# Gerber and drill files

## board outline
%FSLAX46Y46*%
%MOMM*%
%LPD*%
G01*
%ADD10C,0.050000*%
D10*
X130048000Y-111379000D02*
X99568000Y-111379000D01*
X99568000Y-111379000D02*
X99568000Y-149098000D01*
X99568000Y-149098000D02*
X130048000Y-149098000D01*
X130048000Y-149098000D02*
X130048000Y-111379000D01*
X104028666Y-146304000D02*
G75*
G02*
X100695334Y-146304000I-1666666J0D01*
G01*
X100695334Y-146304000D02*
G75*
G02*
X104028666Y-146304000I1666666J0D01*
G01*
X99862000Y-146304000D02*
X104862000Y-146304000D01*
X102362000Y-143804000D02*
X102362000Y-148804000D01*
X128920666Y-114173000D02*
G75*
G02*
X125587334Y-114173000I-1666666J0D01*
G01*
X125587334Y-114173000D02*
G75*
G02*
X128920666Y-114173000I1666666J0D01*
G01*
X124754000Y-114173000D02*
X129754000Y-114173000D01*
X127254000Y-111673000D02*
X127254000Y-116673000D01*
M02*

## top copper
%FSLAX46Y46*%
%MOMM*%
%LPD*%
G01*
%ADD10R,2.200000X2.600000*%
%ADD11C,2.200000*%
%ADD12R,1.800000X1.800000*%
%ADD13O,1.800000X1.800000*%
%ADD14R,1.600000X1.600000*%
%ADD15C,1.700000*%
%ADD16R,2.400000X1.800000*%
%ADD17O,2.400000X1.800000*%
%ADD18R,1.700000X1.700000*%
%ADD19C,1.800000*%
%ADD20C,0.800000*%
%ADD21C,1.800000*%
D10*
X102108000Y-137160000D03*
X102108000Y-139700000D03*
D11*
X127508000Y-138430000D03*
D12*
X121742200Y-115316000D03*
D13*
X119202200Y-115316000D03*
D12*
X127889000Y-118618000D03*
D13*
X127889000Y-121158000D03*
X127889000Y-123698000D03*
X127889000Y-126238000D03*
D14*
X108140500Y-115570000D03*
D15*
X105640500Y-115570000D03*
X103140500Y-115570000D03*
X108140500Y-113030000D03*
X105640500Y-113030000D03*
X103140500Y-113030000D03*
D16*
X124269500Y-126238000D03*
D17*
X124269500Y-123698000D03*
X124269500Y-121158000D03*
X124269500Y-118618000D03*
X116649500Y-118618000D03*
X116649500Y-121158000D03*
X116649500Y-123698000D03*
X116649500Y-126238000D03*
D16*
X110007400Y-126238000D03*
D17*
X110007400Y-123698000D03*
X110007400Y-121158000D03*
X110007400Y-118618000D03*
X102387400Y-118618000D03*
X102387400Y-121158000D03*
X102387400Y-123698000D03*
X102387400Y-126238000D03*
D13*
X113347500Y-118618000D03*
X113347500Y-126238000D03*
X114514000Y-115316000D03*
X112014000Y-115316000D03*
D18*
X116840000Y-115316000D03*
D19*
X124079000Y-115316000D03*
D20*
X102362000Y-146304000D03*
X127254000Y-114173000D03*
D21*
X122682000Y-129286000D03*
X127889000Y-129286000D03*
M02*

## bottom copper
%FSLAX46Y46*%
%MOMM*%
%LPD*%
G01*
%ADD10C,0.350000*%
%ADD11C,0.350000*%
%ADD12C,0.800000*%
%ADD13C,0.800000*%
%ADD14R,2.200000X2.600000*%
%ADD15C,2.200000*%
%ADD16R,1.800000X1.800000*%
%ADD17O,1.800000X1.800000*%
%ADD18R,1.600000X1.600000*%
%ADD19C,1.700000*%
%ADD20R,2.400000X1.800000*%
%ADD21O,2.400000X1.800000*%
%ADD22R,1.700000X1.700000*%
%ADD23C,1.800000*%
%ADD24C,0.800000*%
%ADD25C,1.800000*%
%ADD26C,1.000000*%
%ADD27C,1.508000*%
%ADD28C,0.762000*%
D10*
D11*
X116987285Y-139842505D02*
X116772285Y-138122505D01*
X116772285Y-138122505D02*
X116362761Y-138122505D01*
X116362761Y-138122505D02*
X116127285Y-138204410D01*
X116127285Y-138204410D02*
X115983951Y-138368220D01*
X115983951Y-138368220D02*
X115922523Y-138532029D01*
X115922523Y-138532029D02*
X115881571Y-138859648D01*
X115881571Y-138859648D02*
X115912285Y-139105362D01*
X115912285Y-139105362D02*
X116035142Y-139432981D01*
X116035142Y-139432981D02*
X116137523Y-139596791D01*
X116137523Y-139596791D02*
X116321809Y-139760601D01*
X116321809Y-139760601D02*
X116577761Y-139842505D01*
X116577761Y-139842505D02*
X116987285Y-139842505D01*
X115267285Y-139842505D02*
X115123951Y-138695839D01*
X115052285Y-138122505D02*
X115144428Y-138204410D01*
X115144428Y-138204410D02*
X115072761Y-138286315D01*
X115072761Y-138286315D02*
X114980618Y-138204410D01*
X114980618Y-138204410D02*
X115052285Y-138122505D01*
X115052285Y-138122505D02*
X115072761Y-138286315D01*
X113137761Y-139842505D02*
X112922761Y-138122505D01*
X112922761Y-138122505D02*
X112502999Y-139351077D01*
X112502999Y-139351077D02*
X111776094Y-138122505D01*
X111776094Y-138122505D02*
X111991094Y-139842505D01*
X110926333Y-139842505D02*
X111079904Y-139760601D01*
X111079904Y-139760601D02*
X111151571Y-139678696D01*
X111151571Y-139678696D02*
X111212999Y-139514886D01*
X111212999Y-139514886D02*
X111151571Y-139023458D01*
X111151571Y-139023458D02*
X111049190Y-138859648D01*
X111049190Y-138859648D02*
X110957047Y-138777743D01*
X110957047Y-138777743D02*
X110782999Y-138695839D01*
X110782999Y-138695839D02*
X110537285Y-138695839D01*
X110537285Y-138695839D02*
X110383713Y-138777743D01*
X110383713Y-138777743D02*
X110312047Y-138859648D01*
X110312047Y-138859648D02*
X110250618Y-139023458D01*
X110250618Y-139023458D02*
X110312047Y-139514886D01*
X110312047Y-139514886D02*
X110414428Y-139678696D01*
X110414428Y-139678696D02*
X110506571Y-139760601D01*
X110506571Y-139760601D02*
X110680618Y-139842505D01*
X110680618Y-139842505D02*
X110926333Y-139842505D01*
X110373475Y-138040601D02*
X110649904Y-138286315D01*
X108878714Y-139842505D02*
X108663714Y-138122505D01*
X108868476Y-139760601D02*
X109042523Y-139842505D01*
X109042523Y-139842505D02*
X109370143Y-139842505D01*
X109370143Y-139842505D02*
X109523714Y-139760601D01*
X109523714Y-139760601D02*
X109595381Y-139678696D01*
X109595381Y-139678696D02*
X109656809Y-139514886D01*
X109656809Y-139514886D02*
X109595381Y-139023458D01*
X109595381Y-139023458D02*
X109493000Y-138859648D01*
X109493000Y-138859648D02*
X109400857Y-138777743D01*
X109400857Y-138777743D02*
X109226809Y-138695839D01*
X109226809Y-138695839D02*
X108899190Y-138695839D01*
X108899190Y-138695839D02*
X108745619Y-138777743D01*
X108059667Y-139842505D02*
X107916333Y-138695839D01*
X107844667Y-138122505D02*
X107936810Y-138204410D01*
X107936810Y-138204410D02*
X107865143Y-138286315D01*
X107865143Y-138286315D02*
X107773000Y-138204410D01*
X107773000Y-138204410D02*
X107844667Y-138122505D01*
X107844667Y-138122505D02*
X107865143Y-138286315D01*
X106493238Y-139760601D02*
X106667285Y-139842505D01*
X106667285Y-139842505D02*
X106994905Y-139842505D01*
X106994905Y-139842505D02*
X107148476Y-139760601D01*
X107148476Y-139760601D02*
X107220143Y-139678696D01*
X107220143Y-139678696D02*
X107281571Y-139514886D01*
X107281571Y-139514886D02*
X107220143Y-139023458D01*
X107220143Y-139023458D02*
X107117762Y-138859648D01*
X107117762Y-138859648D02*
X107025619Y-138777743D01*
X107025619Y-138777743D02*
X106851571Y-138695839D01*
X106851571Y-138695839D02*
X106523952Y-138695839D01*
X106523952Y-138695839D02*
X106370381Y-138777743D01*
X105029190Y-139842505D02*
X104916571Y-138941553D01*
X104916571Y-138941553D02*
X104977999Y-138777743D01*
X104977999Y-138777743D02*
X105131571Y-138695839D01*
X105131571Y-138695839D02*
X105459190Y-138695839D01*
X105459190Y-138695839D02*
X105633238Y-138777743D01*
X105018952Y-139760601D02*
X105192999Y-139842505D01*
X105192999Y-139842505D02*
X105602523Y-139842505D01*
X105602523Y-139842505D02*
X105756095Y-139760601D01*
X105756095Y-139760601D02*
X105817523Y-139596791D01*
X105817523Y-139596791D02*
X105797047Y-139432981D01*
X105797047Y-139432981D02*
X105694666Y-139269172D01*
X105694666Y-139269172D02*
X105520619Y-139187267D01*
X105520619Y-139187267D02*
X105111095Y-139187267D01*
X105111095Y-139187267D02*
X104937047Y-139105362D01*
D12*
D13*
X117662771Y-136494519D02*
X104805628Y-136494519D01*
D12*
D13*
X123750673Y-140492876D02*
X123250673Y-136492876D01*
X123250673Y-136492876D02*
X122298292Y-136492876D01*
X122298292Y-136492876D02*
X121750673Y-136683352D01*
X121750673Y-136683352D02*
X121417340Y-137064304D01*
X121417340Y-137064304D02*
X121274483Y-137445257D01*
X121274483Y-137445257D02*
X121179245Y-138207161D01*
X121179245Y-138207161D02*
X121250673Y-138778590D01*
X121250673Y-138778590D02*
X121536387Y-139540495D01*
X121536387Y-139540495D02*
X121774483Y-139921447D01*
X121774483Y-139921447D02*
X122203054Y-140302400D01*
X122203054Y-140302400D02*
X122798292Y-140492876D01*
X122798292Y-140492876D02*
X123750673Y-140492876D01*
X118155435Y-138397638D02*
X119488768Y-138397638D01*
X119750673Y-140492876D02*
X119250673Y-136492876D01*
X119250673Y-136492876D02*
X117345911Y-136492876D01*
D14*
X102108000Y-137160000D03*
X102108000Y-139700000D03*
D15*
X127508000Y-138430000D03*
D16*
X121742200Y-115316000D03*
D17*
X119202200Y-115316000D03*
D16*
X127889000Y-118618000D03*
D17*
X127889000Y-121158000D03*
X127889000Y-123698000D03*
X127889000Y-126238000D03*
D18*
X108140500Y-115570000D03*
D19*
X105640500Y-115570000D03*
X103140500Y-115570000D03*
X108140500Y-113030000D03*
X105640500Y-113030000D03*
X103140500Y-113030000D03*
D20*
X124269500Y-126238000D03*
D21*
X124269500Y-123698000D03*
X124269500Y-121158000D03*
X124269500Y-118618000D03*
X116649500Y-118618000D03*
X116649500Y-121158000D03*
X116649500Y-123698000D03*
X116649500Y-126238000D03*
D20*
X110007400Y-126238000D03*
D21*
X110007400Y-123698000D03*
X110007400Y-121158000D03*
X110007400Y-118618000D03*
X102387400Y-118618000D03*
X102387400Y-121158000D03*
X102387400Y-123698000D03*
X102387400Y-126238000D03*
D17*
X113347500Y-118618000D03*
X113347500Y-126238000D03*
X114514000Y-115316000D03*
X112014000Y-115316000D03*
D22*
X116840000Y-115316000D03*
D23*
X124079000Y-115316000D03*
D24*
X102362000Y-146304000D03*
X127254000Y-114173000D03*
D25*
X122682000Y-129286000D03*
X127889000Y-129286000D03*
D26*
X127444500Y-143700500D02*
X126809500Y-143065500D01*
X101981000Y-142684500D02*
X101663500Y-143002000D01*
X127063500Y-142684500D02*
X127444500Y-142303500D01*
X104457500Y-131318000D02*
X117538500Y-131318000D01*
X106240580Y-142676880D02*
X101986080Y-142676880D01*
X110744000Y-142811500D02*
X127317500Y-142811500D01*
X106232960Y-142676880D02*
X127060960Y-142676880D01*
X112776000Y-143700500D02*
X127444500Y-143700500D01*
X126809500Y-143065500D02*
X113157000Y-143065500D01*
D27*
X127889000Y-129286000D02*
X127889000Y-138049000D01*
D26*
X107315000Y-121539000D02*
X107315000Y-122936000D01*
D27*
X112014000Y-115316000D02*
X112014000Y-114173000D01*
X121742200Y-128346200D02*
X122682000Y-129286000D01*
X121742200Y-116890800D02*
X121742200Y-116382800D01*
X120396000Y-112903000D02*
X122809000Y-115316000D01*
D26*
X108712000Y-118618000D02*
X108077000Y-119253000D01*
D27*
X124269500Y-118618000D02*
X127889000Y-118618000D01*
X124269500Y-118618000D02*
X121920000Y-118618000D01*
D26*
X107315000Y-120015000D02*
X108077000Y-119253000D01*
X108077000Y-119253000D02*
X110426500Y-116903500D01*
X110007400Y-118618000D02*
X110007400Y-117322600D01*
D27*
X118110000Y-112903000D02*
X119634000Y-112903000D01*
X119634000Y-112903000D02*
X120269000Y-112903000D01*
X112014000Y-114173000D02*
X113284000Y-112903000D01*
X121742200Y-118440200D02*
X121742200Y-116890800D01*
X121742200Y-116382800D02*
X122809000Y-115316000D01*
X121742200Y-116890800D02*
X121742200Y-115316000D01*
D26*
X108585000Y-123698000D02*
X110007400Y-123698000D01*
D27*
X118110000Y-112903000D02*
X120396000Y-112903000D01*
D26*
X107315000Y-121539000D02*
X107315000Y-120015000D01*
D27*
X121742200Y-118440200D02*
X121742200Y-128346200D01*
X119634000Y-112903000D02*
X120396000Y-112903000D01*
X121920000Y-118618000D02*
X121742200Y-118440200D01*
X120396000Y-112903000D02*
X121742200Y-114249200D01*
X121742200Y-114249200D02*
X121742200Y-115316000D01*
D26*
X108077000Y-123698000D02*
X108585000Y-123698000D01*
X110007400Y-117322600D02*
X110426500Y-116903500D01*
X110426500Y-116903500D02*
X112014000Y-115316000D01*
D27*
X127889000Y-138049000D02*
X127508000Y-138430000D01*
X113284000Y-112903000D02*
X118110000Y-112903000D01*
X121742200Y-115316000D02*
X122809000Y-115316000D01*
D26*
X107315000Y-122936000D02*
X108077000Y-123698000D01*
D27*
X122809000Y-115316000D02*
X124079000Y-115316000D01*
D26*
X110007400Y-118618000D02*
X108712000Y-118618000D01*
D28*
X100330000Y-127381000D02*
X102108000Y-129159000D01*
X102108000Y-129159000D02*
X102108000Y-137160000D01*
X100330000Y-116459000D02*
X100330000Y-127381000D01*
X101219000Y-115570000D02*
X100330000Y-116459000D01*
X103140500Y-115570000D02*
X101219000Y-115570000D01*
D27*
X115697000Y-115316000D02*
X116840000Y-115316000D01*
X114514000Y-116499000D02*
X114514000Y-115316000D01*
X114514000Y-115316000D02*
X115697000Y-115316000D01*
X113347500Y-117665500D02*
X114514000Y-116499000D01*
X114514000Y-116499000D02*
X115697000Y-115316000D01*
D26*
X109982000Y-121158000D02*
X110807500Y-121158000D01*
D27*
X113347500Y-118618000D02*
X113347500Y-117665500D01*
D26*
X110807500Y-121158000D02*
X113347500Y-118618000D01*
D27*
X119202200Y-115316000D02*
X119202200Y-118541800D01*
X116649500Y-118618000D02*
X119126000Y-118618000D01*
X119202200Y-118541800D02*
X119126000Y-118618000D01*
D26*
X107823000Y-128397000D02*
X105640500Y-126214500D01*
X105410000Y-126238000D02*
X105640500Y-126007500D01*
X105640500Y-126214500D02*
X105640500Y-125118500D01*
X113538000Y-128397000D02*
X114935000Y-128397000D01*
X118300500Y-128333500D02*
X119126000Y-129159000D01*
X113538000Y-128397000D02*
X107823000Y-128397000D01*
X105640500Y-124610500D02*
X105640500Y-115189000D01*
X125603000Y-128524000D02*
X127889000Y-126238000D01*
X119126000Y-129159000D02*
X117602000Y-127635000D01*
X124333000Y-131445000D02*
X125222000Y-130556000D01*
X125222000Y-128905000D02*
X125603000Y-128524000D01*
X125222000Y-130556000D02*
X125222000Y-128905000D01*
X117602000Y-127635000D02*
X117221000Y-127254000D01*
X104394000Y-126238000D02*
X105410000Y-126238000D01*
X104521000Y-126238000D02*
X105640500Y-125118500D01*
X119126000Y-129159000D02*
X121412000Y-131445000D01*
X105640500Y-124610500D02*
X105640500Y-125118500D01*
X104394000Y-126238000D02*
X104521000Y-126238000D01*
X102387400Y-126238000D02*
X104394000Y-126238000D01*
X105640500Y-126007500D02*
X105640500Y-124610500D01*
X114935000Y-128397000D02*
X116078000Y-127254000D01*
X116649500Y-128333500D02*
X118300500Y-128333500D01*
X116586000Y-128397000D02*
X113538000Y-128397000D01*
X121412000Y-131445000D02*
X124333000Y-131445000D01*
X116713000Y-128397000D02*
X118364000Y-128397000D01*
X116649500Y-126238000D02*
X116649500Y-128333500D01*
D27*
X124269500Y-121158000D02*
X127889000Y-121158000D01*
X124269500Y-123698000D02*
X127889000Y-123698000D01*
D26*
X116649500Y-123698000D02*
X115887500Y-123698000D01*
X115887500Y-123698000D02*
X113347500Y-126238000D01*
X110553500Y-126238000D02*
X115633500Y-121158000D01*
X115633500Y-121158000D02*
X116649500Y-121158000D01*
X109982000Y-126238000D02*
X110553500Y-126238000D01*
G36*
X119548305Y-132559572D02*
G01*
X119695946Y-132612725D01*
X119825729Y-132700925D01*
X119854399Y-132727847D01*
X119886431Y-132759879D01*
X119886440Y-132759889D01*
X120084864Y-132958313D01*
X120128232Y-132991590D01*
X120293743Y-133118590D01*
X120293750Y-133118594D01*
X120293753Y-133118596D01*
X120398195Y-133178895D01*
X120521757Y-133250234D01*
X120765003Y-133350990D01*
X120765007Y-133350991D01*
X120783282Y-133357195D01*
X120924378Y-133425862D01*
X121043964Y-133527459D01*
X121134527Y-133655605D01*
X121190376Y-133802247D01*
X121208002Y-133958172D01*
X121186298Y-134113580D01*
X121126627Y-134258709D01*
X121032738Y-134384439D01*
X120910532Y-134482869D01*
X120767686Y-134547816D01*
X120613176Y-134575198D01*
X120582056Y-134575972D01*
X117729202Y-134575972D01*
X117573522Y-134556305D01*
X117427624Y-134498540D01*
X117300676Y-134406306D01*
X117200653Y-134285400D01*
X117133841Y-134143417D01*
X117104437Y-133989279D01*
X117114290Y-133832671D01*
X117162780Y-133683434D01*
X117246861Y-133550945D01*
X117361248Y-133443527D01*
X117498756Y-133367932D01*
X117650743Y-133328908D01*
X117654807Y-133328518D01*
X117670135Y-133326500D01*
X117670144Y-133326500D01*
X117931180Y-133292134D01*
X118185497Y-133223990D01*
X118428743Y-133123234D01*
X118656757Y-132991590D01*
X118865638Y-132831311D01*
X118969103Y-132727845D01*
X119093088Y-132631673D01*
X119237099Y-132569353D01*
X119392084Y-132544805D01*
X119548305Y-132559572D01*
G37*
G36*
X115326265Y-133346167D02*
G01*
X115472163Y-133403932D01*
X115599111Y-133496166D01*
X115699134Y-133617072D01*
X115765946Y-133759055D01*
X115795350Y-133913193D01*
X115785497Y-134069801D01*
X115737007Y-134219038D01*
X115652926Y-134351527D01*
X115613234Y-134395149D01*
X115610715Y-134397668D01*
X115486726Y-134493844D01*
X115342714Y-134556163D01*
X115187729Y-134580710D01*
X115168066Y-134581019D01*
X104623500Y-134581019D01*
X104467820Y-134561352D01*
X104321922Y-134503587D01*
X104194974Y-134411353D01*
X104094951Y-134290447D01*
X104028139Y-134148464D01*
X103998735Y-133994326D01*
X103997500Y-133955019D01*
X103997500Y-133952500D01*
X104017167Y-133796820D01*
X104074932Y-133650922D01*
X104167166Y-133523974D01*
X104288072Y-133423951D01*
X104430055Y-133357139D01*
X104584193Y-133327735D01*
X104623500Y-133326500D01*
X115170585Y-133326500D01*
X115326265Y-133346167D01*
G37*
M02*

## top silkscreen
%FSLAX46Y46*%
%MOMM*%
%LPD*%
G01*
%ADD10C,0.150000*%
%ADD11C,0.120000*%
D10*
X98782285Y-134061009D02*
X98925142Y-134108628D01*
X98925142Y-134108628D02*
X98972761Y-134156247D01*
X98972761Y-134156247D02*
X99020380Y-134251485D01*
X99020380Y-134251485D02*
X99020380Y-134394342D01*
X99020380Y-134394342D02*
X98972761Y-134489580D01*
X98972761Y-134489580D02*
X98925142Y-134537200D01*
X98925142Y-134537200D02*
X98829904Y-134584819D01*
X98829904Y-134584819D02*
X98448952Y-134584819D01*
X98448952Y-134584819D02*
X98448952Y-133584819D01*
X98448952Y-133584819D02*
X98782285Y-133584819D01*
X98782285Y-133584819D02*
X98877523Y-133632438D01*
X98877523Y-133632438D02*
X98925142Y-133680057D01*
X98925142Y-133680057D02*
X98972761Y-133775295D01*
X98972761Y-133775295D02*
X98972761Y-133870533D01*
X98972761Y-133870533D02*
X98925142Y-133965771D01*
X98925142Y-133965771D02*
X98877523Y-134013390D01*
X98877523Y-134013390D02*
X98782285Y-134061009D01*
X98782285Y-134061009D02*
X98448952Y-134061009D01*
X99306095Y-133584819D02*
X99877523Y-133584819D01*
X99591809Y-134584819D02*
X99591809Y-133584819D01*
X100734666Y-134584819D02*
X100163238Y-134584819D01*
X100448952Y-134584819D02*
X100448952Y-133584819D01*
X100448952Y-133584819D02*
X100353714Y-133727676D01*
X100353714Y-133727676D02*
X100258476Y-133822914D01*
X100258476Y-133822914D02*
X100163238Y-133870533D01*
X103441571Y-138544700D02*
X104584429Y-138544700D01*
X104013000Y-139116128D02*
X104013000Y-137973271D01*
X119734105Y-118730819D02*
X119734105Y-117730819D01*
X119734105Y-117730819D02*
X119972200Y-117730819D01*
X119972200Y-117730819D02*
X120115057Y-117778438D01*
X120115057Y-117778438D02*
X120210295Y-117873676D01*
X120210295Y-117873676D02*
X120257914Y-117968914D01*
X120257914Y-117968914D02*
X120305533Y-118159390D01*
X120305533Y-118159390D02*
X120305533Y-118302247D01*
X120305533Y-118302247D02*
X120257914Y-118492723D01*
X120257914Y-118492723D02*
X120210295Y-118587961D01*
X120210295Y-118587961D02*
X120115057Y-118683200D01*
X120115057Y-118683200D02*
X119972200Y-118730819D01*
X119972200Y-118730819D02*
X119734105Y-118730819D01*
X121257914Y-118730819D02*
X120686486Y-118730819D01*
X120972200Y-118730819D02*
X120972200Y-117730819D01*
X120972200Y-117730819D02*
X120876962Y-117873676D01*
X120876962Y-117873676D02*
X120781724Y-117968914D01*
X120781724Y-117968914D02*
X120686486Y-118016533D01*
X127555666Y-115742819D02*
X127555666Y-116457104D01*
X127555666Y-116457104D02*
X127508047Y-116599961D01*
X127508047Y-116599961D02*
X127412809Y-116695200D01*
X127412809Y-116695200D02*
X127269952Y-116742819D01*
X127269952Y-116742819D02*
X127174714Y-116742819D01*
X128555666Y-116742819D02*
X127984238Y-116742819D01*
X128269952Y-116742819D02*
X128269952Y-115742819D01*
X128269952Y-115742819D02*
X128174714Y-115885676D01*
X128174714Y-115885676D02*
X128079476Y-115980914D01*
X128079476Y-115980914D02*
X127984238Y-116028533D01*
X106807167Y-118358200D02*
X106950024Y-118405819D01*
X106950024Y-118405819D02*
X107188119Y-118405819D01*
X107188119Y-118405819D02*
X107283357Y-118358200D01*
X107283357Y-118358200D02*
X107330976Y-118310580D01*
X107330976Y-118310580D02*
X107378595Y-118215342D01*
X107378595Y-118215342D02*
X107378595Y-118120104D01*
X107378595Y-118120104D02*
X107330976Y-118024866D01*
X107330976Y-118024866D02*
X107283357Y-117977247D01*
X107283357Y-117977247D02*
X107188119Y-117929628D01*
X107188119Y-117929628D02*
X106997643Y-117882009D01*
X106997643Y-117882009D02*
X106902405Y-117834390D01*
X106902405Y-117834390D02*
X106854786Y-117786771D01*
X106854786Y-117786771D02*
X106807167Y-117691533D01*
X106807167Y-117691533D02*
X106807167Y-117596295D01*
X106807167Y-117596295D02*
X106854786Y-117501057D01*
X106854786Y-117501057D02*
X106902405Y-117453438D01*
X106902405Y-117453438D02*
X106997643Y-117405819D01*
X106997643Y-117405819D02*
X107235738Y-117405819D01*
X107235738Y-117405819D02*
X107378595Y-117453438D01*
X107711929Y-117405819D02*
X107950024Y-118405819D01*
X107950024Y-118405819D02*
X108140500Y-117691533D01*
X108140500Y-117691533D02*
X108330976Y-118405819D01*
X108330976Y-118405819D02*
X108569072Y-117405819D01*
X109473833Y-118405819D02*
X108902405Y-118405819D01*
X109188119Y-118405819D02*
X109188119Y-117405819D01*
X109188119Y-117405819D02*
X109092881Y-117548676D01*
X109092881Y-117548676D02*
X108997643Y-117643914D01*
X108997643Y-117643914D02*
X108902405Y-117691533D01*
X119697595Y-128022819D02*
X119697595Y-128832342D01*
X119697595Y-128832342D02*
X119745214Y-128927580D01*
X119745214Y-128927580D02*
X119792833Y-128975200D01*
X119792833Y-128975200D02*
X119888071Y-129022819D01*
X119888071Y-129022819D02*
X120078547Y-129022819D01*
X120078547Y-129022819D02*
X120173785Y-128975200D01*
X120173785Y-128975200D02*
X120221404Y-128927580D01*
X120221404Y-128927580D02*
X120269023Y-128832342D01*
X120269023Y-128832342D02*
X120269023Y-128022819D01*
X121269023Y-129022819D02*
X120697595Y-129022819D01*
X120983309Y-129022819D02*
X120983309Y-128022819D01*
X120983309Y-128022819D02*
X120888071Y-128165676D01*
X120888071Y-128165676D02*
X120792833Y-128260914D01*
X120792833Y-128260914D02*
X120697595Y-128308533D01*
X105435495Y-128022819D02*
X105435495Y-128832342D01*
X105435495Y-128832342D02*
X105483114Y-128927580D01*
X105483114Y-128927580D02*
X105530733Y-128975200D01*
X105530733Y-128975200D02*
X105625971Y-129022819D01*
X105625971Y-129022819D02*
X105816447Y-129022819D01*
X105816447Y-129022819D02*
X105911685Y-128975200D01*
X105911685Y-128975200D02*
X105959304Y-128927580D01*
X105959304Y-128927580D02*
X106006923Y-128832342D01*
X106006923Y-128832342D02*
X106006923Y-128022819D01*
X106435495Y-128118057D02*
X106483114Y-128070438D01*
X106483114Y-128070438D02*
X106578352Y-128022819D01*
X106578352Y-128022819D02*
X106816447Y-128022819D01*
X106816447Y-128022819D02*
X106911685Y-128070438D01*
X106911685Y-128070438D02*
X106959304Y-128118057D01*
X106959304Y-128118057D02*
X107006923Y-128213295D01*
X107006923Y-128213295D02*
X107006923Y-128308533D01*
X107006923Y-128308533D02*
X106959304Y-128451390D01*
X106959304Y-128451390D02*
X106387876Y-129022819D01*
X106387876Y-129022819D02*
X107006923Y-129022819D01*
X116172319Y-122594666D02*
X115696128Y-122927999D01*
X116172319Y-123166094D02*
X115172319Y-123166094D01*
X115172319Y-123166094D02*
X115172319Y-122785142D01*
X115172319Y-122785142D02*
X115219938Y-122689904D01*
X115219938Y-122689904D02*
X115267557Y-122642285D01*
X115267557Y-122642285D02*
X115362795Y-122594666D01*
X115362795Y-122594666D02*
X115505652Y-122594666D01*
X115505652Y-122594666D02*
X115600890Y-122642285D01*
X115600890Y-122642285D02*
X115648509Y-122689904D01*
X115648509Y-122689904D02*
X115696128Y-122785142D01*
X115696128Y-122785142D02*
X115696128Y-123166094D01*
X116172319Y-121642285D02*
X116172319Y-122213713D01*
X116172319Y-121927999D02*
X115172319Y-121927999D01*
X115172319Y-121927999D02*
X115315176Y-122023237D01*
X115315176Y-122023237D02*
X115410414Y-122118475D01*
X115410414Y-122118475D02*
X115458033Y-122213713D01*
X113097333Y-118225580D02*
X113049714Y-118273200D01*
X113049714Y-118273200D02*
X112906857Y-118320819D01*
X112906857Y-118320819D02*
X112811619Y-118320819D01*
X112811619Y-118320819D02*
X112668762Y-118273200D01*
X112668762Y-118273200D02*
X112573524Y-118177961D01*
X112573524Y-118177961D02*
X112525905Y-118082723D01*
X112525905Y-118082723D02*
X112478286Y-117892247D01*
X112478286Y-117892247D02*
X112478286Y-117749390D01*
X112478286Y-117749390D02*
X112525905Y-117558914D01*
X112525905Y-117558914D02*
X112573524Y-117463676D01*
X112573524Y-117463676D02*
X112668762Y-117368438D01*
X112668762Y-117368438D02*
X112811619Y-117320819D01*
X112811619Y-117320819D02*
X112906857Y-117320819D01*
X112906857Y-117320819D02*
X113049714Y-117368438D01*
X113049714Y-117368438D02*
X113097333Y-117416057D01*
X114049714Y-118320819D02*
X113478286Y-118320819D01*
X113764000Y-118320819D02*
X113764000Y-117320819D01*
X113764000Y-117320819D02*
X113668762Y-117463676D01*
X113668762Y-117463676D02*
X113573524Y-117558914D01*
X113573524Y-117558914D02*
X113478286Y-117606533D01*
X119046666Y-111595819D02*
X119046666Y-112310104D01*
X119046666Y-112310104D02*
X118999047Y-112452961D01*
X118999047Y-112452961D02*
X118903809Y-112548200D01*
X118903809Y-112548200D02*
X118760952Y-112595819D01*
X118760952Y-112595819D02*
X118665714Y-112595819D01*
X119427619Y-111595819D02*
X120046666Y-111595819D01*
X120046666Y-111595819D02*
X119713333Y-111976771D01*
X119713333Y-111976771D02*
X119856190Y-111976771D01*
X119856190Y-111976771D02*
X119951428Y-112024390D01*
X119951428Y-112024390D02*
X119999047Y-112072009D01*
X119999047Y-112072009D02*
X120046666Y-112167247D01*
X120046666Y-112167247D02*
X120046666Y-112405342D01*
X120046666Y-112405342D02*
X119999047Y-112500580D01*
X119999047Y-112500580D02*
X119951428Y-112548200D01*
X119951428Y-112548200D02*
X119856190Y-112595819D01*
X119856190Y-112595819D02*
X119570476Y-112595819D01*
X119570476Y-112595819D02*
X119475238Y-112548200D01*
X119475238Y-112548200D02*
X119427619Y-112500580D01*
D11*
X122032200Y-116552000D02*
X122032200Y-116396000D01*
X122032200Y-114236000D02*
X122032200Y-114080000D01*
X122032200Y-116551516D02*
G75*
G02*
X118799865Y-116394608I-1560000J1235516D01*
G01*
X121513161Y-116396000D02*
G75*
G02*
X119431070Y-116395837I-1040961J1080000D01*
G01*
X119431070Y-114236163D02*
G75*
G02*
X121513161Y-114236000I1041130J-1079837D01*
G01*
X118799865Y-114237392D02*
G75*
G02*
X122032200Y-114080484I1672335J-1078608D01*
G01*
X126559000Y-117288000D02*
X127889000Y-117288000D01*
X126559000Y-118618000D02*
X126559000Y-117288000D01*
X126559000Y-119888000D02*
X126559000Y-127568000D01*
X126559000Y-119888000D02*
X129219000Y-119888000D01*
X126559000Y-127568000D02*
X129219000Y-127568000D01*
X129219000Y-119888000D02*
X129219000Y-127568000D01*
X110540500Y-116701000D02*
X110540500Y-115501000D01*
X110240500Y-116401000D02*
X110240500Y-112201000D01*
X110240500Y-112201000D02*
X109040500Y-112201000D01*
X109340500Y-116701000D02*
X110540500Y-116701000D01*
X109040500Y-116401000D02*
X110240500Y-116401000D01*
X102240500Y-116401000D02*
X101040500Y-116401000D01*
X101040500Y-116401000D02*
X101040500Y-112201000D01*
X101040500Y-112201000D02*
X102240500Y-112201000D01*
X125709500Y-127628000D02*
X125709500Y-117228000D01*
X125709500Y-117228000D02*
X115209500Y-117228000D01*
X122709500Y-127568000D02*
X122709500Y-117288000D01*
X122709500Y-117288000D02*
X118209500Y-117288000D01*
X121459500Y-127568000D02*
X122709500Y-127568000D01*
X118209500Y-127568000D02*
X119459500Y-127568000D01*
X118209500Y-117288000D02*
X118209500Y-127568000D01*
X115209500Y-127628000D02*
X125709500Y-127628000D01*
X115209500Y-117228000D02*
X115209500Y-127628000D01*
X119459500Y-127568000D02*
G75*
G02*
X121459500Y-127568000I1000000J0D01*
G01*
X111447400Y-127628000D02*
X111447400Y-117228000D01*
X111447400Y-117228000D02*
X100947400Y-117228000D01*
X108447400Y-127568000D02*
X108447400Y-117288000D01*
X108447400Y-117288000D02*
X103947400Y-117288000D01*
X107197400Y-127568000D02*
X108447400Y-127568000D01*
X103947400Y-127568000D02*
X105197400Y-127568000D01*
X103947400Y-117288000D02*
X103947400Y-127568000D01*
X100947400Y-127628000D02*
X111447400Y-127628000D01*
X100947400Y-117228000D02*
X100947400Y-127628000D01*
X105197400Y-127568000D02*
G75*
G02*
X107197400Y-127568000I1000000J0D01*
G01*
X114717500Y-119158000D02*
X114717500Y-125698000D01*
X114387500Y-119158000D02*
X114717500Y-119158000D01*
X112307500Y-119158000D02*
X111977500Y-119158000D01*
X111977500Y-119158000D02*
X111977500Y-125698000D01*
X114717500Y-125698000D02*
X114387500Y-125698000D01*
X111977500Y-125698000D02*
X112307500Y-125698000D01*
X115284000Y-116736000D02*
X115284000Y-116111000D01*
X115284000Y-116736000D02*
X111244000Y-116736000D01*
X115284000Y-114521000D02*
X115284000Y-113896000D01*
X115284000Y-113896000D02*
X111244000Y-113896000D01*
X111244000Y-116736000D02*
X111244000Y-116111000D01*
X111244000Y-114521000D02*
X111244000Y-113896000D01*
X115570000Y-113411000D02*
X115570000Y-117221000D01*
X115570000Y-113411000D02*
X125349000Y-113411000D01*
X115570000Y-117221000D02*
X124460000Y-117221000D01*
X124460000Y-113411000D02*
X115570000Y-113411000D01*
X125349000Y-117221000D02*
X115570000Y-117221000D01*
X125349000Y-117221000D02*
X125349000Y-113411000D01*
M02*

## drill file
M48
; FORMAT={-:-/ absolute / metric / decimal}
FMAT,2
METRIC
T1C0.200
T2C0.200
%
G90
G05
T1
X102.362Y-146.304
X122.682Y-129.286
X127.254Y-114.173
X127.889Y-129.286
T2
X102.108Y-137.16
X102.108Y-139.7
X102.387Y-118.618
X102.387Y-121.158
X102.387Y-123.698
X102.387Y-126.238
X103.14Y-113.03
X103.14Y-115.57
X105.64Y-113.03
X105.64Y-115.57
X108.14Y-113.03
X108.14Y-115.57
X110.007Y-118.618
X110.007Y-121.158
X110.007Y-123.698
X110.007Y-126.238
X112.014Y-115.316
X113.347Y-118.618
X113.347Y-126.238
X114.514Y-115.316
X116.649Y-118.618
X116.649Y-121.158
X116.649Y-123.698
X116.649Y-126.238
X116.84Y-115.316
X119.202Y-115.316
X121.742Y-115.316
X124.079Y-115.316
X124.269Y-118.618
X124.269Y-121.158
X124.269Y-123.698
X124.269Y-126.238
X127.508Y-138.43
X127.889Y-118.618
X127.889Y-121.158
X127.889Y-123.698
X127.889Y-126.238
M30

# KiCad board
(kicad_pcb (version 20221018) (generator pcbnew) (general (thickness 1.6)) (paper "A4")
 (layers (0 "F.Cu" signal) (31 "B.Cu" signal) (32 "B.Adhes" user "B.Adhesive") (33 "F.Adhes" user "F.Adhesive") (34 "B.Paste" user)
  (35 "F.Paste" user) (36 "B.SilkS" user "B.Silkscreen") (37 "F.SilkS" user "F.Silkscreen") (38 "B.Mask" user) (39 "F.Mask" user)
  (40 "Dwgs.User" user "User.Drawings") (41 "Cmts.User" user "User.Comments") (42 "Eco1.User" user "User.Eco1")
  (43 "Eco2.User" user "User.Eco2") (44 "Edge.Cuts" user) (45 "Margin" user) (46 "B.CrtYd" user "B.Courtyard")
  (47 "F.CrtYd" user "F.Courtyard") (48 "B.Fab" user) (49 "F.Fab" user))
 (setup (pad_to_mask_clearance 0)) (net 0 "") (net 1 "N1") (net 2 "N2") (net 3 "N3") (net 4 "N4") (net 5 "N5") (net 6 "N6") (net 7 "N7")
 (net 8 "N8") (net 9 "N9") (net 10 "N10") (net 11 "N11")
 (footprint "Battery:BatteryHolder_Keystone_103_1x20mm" (layer "F.Cu") (at 99.568 138.43)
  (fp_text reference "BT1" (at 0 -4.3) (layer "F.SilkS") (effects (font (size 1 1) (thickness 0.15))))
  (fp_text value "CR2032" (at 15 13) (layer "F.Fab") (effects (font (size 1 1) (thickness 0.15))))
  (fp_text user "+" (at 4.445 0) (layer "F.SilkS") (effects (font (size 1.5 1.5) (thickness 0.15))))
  (pad "1" thru_hole rect (at 2.54 -1.27) (size 2.2 2.6) (drill 0.2) (layers "*.Cu" "*.Mask") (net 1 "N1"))
  (pad "1" thru_hole rect (at 2.54 1.27) (size 2.2 2.6) (drill 0.2) (layers "*.Cu" "*.Mask") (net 1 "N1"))
  (pad "2" thru_hole circle (at 27.94 0) (size 2.2 2.2) (drill 0.2) (layers "*.Cu" "*.Mask") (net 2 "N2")))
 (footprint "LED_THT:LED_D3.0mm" (layer "F.Cu") (at 121.7422 115.316 180)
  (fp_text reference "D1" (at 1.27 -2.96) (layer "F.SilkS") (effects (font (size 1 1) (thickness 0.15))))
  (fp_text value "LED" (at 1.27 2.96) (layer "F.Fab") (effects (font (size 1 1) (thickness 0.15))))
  (fp_line (start -0.29 -1.236) (end -0.29 -1.08) (stroke (width 0.12) (type solid)) (layer "F.SilkS"))
  (fp_line (start -0.29 1.08) (end -0.29 1.236) (stroke (width 0.12) (type solid)) (layer "F.SilkS"))
  (fp_arc (start -0.29 -1.235516) (mid 1.366487 -1.987659) (end 2.942335 -1.078608) (stroke (width 0.12) (type solid)) (layer "F.SilkS"))
  (fp_arc (start 0.229039 -1.08) (mid 1.270117 -1.5) (end 2.31113 -1.079837) (stroke (width 0.12) (type solid)) (layer "F.SilkS"))
  (fp_arc (start 2.31113 1.079837) (mid 1.270117 1.5) (end 0.229039 1.08) (stroke (width 0.12) (type solid)) (layer "F.SilkS"))
  (fp_arc (start 2.942335 1.078608) (mid 1.366487 1.987659) (end -0.29 1.235516) (stroke (width 0.12) (type solid)) (layer "F.SilkS"))
  (pad "1" thru_hole rect (at 0 0 180) (size 1.8 1.8) (drill 0.2) (layers "*.Cu" "*.Mask") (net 2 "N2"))
  (pad "2" thru_hole oval (at 2.54 0 180) (size 1.8 1.8) (drill 0.2) (layers "*.Cu" "*.Mask") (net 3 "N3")))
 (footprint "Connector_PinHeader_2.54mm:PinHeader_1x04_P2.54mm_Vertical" (layer "F.Cu") (at 127.889 118.618)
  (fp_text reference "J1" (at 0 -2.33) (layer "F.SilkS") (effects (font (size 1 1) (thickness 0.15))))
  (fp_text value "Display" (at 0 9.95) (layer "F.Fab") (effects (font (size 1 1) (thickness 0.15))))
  (fp_line (start -1.33 -1.33) (end 0 -1.33) (stroke (width 0.12) (type solid)) (layer "F.SilkS"))
  (fp_line (start -1.33 0) (end -1.33 -1.33) (stroke (width 0.12) (type solid)) (layer "F.SilkS"))
  (fp_line (start -1.33 1.27) (end -1.33 8.95) (stroke (width 0.12) (type solid)) (layer "F.SilkS"))
  (fp_line (start -1.33 1.27) (end 1.33 1.27) (stroke (width 0.12) (type solid)) (layer "F.SilkS"))
  (fp_line (start -1.33 8.95) (end 1.33 8.95) (stroke (width 0.12) (type solid)) (layer "F.SilkS"))
  (fp_line (start 1.33 1.27) (end 1.33 8.95) (stroke (width 0.12) (type solid)) (layer "F.SilkS"))
  (pad "1" thru_hole rect (at 0 0) (size 1.8 1.8) (drill 0.2) (layers "*.Cu" "*.Mask") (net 2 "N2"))
  (pad "2" thru_hole oval (at 0 2.54) (size 1.8 1.8) (drill 0.2) (layers "*.Cu" "*.Mask") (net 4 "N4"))
  (pad "3" thru_hole oval (at 0 5.08) (size 1.8 1.8) (drill 0.2) (layers "*.Cu" "*.Mask") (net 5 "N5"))
  (pad "4" thru_hole oval (at 0 7.62) (size 1.8 1.8) (drill 0.2) (layers "*.Cu" "*.Mask") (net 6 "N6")))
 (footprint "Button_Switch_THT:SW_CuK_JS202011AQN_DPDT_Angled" (layer "F.Cu") (at 108.1405 115.951 180)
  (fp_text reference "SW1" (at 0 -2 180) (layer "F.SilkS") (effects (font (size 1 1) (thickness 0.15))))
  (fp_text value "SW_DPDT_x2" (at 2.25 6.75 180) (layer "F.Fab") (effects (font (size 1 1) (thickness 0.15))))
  (fp_line (start -2.4 -0.75) (end -2.4 0.45) (stroke (width 0.12) (type solid)) (layer "F.SilkS"))
  (fp_line (start -2.1 -0.45) (end -2.1 3.75) (stroke (width 0.12) (type solid)) (layer "F.SilkS"))
  (fp_line (start -2.1 3.75) (end -0.9 3.75) (stroke (width 0.12) (type solid)) (layer "F.SilkS"))
  (fp_line (start -1.2 -0.75) (end -2.4 -0.75) (stroke (width 0.12) (type solid)) (layer "F.SilkS"))
  (fp_line (start -0.9 -0.45) (end -2.1 -0.45) (stroke (width 0.12) (type solid)) (layer "F.SilkS"))
  (fp_line (start 5.9 -0.45) (end 7.1 -0.45) (stroke (width 0.12) (type solid)) (layer "F.SilkS"))
  (fp_line (start 7.1 -0.45) (end 7.1 3.75) (stroke (width 0.12) (type solid)) (layer "F.SilkS"))
  (fp_line (start 7.1 3.75) (end 5.9 3.75) (stroke (width 0.12) (type solid)) (layer "F.SilkS"))
  (pad "1" thru_hole rect (at 0 0.381 180) (size 1.6 1.6) (drill 0.2) (layers "*.Cu" "*.Mask") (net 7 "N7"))
  (pad "2" thru_hole circle (at 2.5 0.381 180) (size 1.7 1.7) (drill 0.2) (layers "*.Cu" "*.Mask") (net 6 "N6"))
  (pad "3" thru_hole circle (at 5 0.381 180) (size 1.7 1.7) (drill 0.2) (layers "*.Cu" "*.Mask") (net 1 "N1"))
  (pad "4" thru_hole circle (at 0 2.921 180) (size 1.7 1.7) (drill 0.2) (layers "*.Cu" "*.Mask"))
  (pad "5" thru_hole circle (at 2.5 2.921 180) (size 1.7 1.7) (drill 0.2) (layers "*.Cu" "*.Mask"))
  (pad "6" thru_hole circle (at 5 2.921 180) (size 1.7 1.7) (drill 0.2) (layers "*.Cu" "*.Mask")))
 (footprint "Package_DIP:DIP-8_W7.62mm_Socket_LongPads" (layer "F.Cu") (at 124.2695 126.238 180)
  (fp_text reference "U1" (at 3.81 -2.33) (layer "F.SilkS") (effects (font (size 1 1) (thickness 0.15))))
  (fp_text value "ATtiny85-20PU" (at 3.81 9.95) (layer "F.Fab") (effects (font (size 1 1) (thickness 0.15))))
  (fp_line (start -1.44 -1.39) (end -1.44 9.01) (stroke (width 0.12) (type solid)) (layer "F.SilkS"))
  (fp_line (start -1.44 9.01) (end 9.06 9.01) (stroke (width 0.12) (type solid)) (layer "F.SilkS"))
  (fp_line (start 1.56 -1.33) (end 1.56 8.95) (stroke (width 0.12) (type solid)) (layer "F.SilkS"))
  (fp_line (start 1.56 8.95) (end 6.06 8.95) (stroke (width 0.12) (type solid)) (layer "F.SilkS"))
  (fp_line (start 2.81 -1.33) (end 1.56 -1.33) (stroke (width 0.12) (type solid)) (layer "F.SilkS"))
  (fp_line (start 6.06 -1.33) (end 4.81 -1.33) (stroke (width 0.12) (type solid)) (layer "F.SilkS"))
  (fp_line (start 6.06 8.95) (end 6.06 -1.33) (stroke (width 0.12) (type solid)) (layer "F.SilkS"))
  (fp_line (start 9.06 -1.39) (end -1.44 -1.39) (stroke (width 0.12) (type solid)) (layer "F.SilkS"))
  (fp_line (start 9.06 9.01) (end 9.06 -1.39) (stroke (width 0.12) (type solid)) (layer "F.SilkS"))
  (fp_arc (start 4.81 -1.33) (mid 3.81 -0.33) (end 2.81 -1.33) (stroke (width 0.12) (type solid)) (layer "F.SilkS"))
  (pad "1" thru_hole rect (at 0 0 180) (size 2.4 1.8) (drill 0.2) (layers "*.Cu" "*.Mask") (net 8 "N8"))
  (pad "2" thru_hole oval (at 0 2.54 180) (size 2.4 1.8) (drill 0.2) (layers "*.Cu" "*.Mask") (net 5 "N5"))
  (pad "3" thru_hole oval (at 0 5.08 180) (size 2.4 1.8) (drill 0.2) (layers "*.Cu" "*.Mask") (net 4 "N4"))
  (pad "4" thru_hole oval (at 0 7.62 180) (size 2.4 1.8) (drill 0.2) (layers "*.Cu" "*.Mask") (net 2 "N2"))
  (pad "5" thru_hole oval (at 7.62 7.62 180) (size 2.4 1.8) (drill 0.2) (layers "*.Cu" "*.Mask") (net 3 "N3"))
  (pad "6" thru_hole oval (at 7.62 5.08 180) (size 2.4 1.8) (drill 0.2) (layers "*.Cu" "*.Mask") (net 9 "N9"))
  (pad "7" thru_hole oval (at 7.62 2.54 180) (size 2.4 1.8) (drill 0.2) (layers "*.Cu" "*.Mask") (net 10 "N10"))
  (pad "8" thru_hole oval (at 7.62 0 180) (size 2.4 1.8) (drill 0.2) (layers "*.Cu" "*.Mask") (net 6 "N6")))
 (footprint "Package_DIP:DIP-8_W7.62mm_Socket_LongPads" (layer "F.Cu") (at 110.0074 126.238 180)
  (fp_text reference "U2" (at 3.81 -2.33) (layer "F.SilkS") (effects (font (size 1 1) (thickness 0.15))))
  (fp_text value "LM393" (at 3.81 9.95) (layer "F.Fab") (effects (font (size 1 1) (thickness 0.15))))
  (fp_line (start -1.44 -1.39) (end -1.44 9.01) (stroke (width 0.12) (type solid)) (layer "F.SilkS"))
  (fp_line (start -1.44 9.01) (end 9.06 9.01) (stroke (width 0.12) (type solid)) (layer "F.SilkS"))
  (fp_line (start 1.56 -1.33) (end 1.56 8.95) (stroke (width 0.12) (type solid)) (layer "F.SilkS"))
  (fp_line (start 1.56 8.95) (end 6.06 8.95) (stroke (width 0.12) (type solid)) (layer "F.SilkS"))
  (fp_line (start 2.81 -1.33) (end 1.56 -1.33) (stroke (width 0.12) (type solid)) (layer "F.SilkS"))
  (fp_line (start 6.06 -1.33) (end 4.81 -1.33) (stroke (width 0.12) (type solid)) (layer "F.SilkS"))
  (fp_line (start 6.06 8.95) (end 6.06 -1.33) (stroke (width 0.12) (type solid)) (layer "F.SilkS"))
  (fp_line (start 9.06 -1.39) (end -1.44 -1.39) (stroke (width 0.12) (type solid)) (layer "F.SilkS"))
  (fp_line (start 9.06 9.01) (end 9.06 -1.39) (stroke (width 0.12) (type solid)) (layer "F.SilkS"))
  (fp_arc (start 4.81 -1.33) (mid 3.81 -0.33) (end 2.81 -1.33) (stroke (width 0.12) (type solid)) (layer "F.SilkS"))
  (pad "1" thru_hole rect (at 0 0 180) (size 2.4 1.8) (drill 0.2) (layers "*.Cu" "*.Mask") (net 9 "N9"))
  (pad "2" thru_hole oval (at 0 2.54 180) (size 2.4 1.8) (drill 0.2) (layers "*.Cu" "*.Mask") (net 2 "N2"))
  (pad "3" thru_hole oval (at 0 5.08 180) (size 2.4 1.8) (drill 0.2) (layers "*.Cu" "*.Mask") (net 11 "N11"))
  (pad "4" thru_hole oval (at 0 7.62 180) (size 2.4 1.8) (drill 0.2) (layers "*.Cu" "*.Mask") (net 2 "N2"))
  (pad "5" thru_hole oval (at 7.62 7.62 180) (size 2.4 1.8) (drill 0.2) (layers "*.Cu" "*.Mask"))
  (pad "6" thru_hole oval (at 7.62 5.08 180) (size 2.4 1.8) (drill 0.2) (layers "*.Cu" "*.Mask"))
  (pad "7" thru_hole oval (at 7.62 2.54 180) (size 2.4 1.8) (drill 0.2) (layers "*.Cu" "*.Mask"))
  (pad "8" thru_hole oval (at 7.62 0 180) (size 2.4 1.8) (drill 0.2) (layers "*.Cu" "*.Mask") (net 6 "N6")))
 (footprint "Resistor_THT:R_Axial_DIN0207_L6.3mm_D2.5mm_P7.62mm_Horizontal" (layer "F.Cu") (at 113.3475 118.618 -90)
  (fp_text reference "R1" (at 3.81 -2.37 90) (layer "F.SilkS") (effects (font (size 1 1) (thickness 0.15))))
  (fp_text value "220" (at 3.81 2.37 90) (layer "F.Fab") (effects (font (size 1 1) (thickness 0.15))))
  (fp_line (start 0.54 -1.37) (end 7.08 -1.37) (stroke (width 0.12) (type solid)) (layer "F.SilkS"))
  (fp_line (start 0.54 -1.04) (end 0.54 -1.37) (stroke (width 0.12) (type solid)) (layer "F.SilkS"))
  (fp_line (start 0.54 1.04) (end 0.54 1.37) (stroke (width 0.12) (type solid)) (layer "F.SilkS"))
  (fp_line (start 0.54 1.37) (end 7.08 1.37) (stroke (width 0.12) (type solid)) (layer "F.SilkS"))
  (fp_line (start 7.08 -1.37) (end 7.08 -1.04) (stroke (width 0.12) (type solid)) (layer "F.SilkS"))
  (fp_line (start 7.08 1.37) (end 7.08 1.04) (stroke (width 0.12) (type solid)) (layer "F.SilkS"))
  (pad "1" thru_hole oval (at 0 0 270) (size 1.8 1.8) (drill 0.2) (layers "*.Cu" "*.Mask") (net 11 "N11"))
  (pad "2" thru_hole oval (at 7.62 0 270) (size 1.8 1.8) (drill 0.2) (layers "*.Cu" "*.Mask") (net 10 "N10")))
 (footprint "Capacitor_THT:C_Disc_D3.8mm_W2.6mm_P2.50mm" (layer "F.Cu") (at 114.514 115.316 180)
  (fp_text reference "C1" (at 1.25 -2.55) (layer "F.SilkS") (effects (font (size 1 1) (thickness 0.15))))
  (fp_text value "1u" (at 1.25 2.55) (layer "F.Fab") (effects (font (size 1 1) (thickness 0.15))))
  (fp_line (start -0.77 -1.42) (end -0.77 -0.795) (stroke (width 0.12) (type solid)) (layer "F.SilkS"))
  (fp_line (start -0.77 -1.42) (end 3.27 -1.42) (stroke (width 0.12) (type solid)) (layer "F.SilkS"))
  (fp_line (start -0.77 0.795) (end -0.77 1.42) (stroke (width 0.12) (type solid)) (layer "F.SilkS"))
  (fp_line (start -0.77 1.42) (end 3.27 1.42) (stroke (width 0.12) (type solid)) (layer "F.SilkS"))
  (fp_line (start 3.27 -1.42) (end 3.27 -0.795) (stroke (width 0.12) (type solid)) (layer "F.SilkS"))
  (fp_line (start 3.27 0.795) (end 3.27 1.42) (stroke (width 0.12) (type solid)) (layer "F.SilkS"))
  (pad "1" thru_hole oval (at 0 0 180) (size 1.8 1.8) (drill 0.2) (layers "*.Cu" "*.Mask") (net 11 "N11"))
  (pad "2" thru_hole oval (at 2.5 0 180) (size 1.8 1.8) (drill 0.2) (layers "*.Cu" "*.Mask") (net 2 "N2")))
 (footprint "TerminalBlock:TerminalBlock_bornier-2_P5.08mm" (layer "F.Cu") (at 116.84 115.316)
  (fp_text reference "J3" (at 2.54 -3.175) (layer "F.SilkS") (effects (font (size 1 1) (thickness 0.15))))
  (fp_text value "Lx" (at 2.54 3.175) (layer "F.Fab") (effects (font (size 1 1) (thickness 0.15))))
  (fp_line (start -1.27 -1.905) (end -1.27 1.905) (stroke (width 0.12) (type solid)) (layer "F.SilkS"))
  (fp_line (start -1.27 -1.905) (end 8.509 -1.905) (stroke (width 0.12) (type solid)) (layer "F.SilkS"))
  (fp_line (start -1.27 1.905) (end 7.62 1.905) (stroke (width 0.12) (type solid)) (layer "F.SilkS"))
  (fp_line (start 7.62 -1.905) (end -1.27 -1.905) (stroke (width 0.12) (type solid)) (layer "F.SilkS"))
  (fp_line (start 8.509 1.905) (end -1.27 1.905) (stroke (width 0.12) (type solid)) (layer "F.SilkS"))
  (fp_line (start 8.509 1.905) (end 8.509 -1.905) (stroke (width 0.12) (type solid)) (layer "F.SilkS"))
  (pad "1" thru_hole rect (at 0 0) (size 1.7 1.7) (drill 0.2) (layers "*.Cu" "*.Mask") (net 11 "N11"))
  (pad "2" thru_hole circle (at 7.239 0) (size 1.8 1.8) (drill 0.2) (layers "*.Cu" "*.Mask") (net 2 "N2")))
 (gr_line (start 130.048 111.379) (end 99.568 111.379) (stroke (width 0.05) (type solid)) (layer "Edge.Cuts"))
 (gr_line (start 99.568 111.379) (end 99.568 149.098) (stroke (width 0.05) (type solid)) (layer "Edge.Cuts"))
 (gr_line (start 99.568 149.098) (end 130.048 149.098) (stroke (width 0.05) (type solid)) (layer "Edge.Cuts"))
 (gr_line (start 130.048 149.098) (end 130.048 111.379) (stroke (width 0.05) (type solid)) (layer "Edge.Cuts"))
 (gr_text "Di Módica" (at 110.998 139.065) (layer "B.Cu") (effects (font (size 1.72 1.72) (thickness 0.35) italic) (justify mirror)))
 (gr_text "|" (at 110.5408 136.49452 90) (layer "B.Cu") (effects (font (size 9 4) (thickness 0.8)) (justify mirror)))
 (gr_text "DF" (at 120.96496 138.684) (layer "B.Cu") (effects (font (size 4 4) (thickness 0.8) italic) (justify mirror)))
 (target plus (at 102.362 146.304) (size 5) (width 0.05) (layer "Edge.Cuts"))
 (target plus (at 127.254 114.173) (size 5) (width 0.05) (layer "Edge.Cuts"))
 (via (at 102.362 146.304) (size 0.8) (drill 0.2) (layers "F.Cu" "B.Cu") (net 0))
 (via (at 127.254 114.173) (size 0.8) (drill 0.2) (layers "F.Cu" "B.Cu") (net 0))
 (segment (start 127.4445 143.7005) (end 126.8095 143.0655) (width 1) (layer "B.Cu") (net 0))
 (segment (start 101.981 142.6845) (end 101.6635 143.002) (width 1) (layer "B.Cu") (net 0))
 (segment (start 127.0635 142.6845) (end 127.4445 142.3035) (width 1) (layer "B.Cu") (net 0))
 (segment (start 104.4575 131.318) (end 117.5385 131.318) (width 1) (layer "B.Cu") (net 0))
 (segment (start 106.24058 142.67688) (end 101.98608 142.67688) (width 1) (layer "B.Cu") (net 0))
 (segment (start 110.744 142.8115) (end 127.3175 142.8115) (width 1) (layer "B.Cu") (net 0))
 (segment (start 106.23296 142.67688) (end 127.06096 142.67688) (width 1) (layer "B.Cu") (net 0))
 (segment (start 112.776 143.7005) (end 127.4445 143.7005) (width 1) (layer "B.Cu") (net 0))
 (segment (start 126.8095 143.0655) (end 113.157 143.0655) (width 1) (layer "B.Cu") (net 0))
 (via (at 122.682 129.286) (size 1.8) (drill 0.2) (layers "F.Cu" "B.Cu") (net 2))
 (via (at 127.889 129.286) (size 1.8) (drill 0.2) (layers "F.Cu" "B.Cu") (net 2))
 (segment (start 127.889 129.286) (end 127.889 138.049) (width 1.508) (layer "B.Cu") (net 2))
 (segment (start 107.315 121.539) (end 107.315 122.936) (width 1) (layer "B.Cu") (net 2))
 (segment (start 112.014 115.316) (end 112.014 114.173) (width 1.508) (layer "B.Cu") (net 2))
 (segment (start 121.7422 128.3462) (end 122.682 129.286) (width 1.508) (layer "B.Cu") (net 2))
 (segment (start 121.7422 116.8908) (end 121.7422 116.3828) (width 1.508) (layer "B.Cu") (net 2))
 (segment (start 120.396 112.903) (end 122.809 115.316) (width 1.508) (layer "B.Cu") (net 2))
 (segment (start 108.712 118.618) (end 108.077 119.253) (width 1) (layer "B.Cu") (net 2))
 (segment (start 124.2695 118.618) (end 127.889 118.618) (width 1.508) (layer "B.Cu") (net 2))
 (segment (start 124.2695 118.618) (end 121.92 118.618) (width 1.508) (layer "B.Cu") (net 2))
 (segment (start 107.315 120.015) (end 108.077 119.253) (width 1) (layer "B.Cu") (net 2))
 (segment (start 108.077 119.253) (end 110.4265 116.9035) (width 1) (layer "B.Cu") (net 2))
 (segment (start 110.0074 118.618) (end 110.0074 117.3226) (width 1) (layer "B.Cu") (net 2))
 (segment (start 118.11 112.903) (end 119.634 112.903) (width 1.508) (layer "B.Cu") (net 2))
 (segment (start 119.634 112.903) (end 120.269 112.903) (width 1.508) (layer "B.Cu") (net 2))
 (segment (start 112.014 114.173) (end 113.284 112.903) (width 1.508) (layer "B.Cu") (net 2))
 (segment (start 121.7422 118.4402) (end 121.7422 116.8908) (width 1.508) (layer "B.Cu") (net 2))
 (segment (start 121.7422 116.3828) (end 122.809 115.316) (width 1.508) (layer "B.Cu") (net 2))
 (segment (start 121.7422 116.8908) (end 121.7422 115.316) (width 1.508) (layer "B.Cu") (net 2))
 (segment (start 108.585 123.698) (end 110.0074 123.698) (width 1) (layer "B.Cu") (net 2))
 (segment (start 118.11 112.903) (end 120.396 112.903) (width 1.508) (layer "B.Cu") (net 2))
 (segment (start 107.315 121.539) (end 107.315 120.015) (width 1) (layer "B.Cu") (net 2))
 (segment (start 121.7422 118.4402) (end 121.7422 128.3462) (width 1.508) (layer "B.Cu") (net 2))
 (segment (start 119.634 112.903) (end 120.396 112.903) (width 1.508) (layer "B.Cu") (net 2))
 (segment (start 121.92 118.618) (end 121.7422 118.4402) (width 1.508) (layer "B.Cu") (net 2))
 (segment (start 120.396 112.903) (end 121.7422 114.2492) (width 1.508) (layer "B.Cu") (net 2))
 (segment (start 121.7422 114.2492) (end 121.7422 115.316) (width 1.508) (layer "B.Cu") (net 2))
 (segment (start 108.077 123.698) (end 108.585 123.698) (width 1) (layer "B.Cu") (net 2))
 (segment (start 110.0074 117.3226) (end 110.4265 116.9035) (width 1) (layer "B.Cu") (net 2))
 (segment (start 110.4265 116.9035) (end 112.014 115.316) (width 1) (layer "B.Cu") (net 2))
 (segment (start 127.889 138.049) (end 127.508 138.43) (width 1.508) (layer "B.Cu") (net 2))
 (segment (start 113.284 112.903) (end 118.11 112.903) (width 1.508) (layer "B.Cu") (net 2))
 (segment (start 121.7422 115.316) (end 122.809 115.316) (width 1.508) (layer "B.Cu") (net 2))
 (segment (start 107.315 122.936) (end 108.077 123.698) (width 1) (layer "B.Cu") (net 2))
 (segment (start 122.809 115.316) (end 124.079 115.316) (width 1.508) (layer "B.Cu") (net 2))
 (segment (start 110.0074 118.618) (end 108.712 118.618) (width 1) (layer "B.Cu") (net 2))
 (segment (start 100.33 127.381) (end 102.108 129.159) (width 0.762) (layer "B.Cu") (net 1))
 (segment (start 102.108 129.159) (end 102.108 137.16) (width 0.762) (layer "B.Cu") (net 1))
 (segment (start 100.33 116.459) (end 100.33 127.381) (width 0.762) (layer "B.Cu") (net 1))
 (segment (start 101.219 115.57) (end 100.33 116.459) (width 0.762) (layer "B.Cu") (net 1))
 (segment (start 103.1405 115.57) (end 101.219 115.57) (width 0.762) (layer "B.Cu") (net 1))
 (segment (start 115.697 115.316) (end 116.84 115.316) (width 1.508) (layer "B.Cu") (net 11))
 (segment (start 114.514 116.499) (end 114.514 115.316) (width 1.508) (layer "B.Cu") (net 11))
 (segment (start 114.514 115.316) (end 115.697 115.316) (width 1.508) (layer "B.Cu") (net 11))
 (segment (start 113.3475 117.6655) (end 114.514 116.499) (width 1.508) (layer "B.Cu") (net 11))
 (segment (start 114.514 116.499) (end 115.697 115.316) (width 1.508) (layer "B.Cu") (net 11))
 (segment (start 109.982 121.158) (end 110.8075 121.158) (width 1) (layer "B.Cu") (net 11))
 (segment (start 113.3475 118.618) (end 113.3475 117.6655) (width 1.508) (layer "B.Cu") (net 11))
 (segment (start 110.8075 121.158) (end 113.3475 118.618) (width 1) (layer "B.Cu") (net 11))
 (segment (start 119.2022 115.316) (end 119.2022 118.5418) (width 1.508) (layer "B.Cu") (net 3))
 (segment (start 116.6495 118.618) (end 119.126 118.618) (width 1.508) (layer "B.Cu") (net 3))
 (segment (start 119.2022 118.5418) (end 119.126 118.618) (width 1.508) (layer "B.Cu") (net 3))
 (segment (start 107.823 128.397) (end 105.6405 126.2145) (width 1) (layer "B.Cu") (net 6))
 (segment (start 105.41 126.238) (end 105.6405 126.0075) (width 1) (layer "B.Cu") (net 6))
 (segment (start 105.6405 126.2145) (end 105.6405 125.1185) (width 1) (layer "B.Cu") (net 6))
 (segment (start 113.538 128.397) (end 114.935 128.397) (width 1) (layer "B.Cu") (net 6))
 (segment (start 118.3005 128.3335) (end 119.126 129.159) (width 1) (layer "B.Cu") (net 6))
 (segment (start 113.538 128.397) (end 107.823 128.397) (width 1) (layer "B.Cu") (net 6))
 (segment (start 105.6405 124.6105) (end 105.6405 115.189) (width 1) (layer "B.Cu") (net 6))
 (segment (start 125.603 128.524) (end 127.889 126.238) (width 1) (layer "B.Cu") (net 6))
 (segment (start 119.126 129.159) (end 117.602 127.635) (width 1) (layer "B.Cu") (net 6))
 (segment (start 124.333 131.445) (end 125.222 130.556) (width 1) (layer "B.Cu") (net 6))
 (segment (start 125.222 128.905) (end 125.603 128.524) (width 1) (layer "B.Cu") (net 6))
 (segment (start 125.222 130.556) (end 125.222 128.905) (width 1) (layer "B.Cu") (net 6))
 (segment (start 117.602 127.635) (end 117.221 127.254) (width 1) (layer "B.Cu") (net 6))
 (segment (start 104.394 126.238) (end 105.41 126.238) (width 1) (layer "B.Cu") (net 6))
 (segment (start 104.521 126.238) (end 105.6405 125.1185) (width 1) (layer "B.Cu") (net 6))
 (segment (start 119.126 129.159) (end 121.412 131.445) (width 1) (layer "B.Cu") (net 6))
 (segment (start 105.6405 124.6105) (end 105.6405 125.1185) (width 1) (layer "B.Cu") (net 6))
 (segment (start 104.394 126.238) (end 104.521 126.238) (width 1) (layer "B.Cu") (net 6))
 (segment (start 102.3874 126.238) (end 104.394 126.238) (width 1) (layer "B.Cu") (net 6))
 (segment (start 105.6405 126.0075) (end 105.6405 124.6105) (width 1) (layer "B.Cu") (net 6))
 (segment (start 114.935 128.397) (end 116.078 127.254) (width 1) (layer "B.Cu") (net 6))
 (segment (start 116.6495 128.3335) (end 118.3005 128.3335) (width 1) (layer "B.Cu") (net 6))
 (segment (start 116.586 128.397) (end 113.538 128.397) (width 1) (layer "B.Cu") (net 6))
 (segment (start 121.412 131.445) (end 124.333 131.445) (width 1) (layer "B.Cu") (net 6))
 (segment (start 116.713 128.397) (end 118.364 128.397) (width 1) (layer "B.Cu") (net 6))
 (segment (start 116.6495 126.238) (end 116.6495 128.3335) (width 1) (layer "B.Cu") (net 6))
 (segment (start 124.2695 121.158) (end 127.889 121.158) (width 1.508) (layer "B.Cu") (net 4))
 (segment (start 124.2695 123.698) (end 127.889 123.698) (width 1.508) (layer "B.Cu") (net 5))
 (segment (start 116.6495 123.698) (end 115.8875 123.698) (width 1) (layer "B.Cu") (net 10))
 (segment (start 115.8875 123.698) (end 113.3475 126.238) (width 1) (layer "B.Cu") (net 10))
 (segment (start 110.5535 126.238) (end 115.6335 121.158) (width 1) (layer "B.Cu") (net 9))
 (segment (start 115.6335 121.158) (end 116.6495 121.158) (width 1) (layer "B.Cu") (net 9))
 (segment (start 109.982 126.238) (end 110.5535 126.238) (width 1) (layer "B.Cu") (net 9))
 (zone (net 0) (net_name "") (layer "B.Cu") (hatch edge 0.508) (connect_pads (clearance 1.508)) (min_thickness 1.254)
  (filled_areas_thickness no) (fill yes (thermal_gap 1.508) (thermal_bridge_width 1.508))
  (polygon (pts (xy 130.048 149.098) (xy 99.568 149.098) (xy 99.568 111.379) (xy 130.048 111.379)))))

